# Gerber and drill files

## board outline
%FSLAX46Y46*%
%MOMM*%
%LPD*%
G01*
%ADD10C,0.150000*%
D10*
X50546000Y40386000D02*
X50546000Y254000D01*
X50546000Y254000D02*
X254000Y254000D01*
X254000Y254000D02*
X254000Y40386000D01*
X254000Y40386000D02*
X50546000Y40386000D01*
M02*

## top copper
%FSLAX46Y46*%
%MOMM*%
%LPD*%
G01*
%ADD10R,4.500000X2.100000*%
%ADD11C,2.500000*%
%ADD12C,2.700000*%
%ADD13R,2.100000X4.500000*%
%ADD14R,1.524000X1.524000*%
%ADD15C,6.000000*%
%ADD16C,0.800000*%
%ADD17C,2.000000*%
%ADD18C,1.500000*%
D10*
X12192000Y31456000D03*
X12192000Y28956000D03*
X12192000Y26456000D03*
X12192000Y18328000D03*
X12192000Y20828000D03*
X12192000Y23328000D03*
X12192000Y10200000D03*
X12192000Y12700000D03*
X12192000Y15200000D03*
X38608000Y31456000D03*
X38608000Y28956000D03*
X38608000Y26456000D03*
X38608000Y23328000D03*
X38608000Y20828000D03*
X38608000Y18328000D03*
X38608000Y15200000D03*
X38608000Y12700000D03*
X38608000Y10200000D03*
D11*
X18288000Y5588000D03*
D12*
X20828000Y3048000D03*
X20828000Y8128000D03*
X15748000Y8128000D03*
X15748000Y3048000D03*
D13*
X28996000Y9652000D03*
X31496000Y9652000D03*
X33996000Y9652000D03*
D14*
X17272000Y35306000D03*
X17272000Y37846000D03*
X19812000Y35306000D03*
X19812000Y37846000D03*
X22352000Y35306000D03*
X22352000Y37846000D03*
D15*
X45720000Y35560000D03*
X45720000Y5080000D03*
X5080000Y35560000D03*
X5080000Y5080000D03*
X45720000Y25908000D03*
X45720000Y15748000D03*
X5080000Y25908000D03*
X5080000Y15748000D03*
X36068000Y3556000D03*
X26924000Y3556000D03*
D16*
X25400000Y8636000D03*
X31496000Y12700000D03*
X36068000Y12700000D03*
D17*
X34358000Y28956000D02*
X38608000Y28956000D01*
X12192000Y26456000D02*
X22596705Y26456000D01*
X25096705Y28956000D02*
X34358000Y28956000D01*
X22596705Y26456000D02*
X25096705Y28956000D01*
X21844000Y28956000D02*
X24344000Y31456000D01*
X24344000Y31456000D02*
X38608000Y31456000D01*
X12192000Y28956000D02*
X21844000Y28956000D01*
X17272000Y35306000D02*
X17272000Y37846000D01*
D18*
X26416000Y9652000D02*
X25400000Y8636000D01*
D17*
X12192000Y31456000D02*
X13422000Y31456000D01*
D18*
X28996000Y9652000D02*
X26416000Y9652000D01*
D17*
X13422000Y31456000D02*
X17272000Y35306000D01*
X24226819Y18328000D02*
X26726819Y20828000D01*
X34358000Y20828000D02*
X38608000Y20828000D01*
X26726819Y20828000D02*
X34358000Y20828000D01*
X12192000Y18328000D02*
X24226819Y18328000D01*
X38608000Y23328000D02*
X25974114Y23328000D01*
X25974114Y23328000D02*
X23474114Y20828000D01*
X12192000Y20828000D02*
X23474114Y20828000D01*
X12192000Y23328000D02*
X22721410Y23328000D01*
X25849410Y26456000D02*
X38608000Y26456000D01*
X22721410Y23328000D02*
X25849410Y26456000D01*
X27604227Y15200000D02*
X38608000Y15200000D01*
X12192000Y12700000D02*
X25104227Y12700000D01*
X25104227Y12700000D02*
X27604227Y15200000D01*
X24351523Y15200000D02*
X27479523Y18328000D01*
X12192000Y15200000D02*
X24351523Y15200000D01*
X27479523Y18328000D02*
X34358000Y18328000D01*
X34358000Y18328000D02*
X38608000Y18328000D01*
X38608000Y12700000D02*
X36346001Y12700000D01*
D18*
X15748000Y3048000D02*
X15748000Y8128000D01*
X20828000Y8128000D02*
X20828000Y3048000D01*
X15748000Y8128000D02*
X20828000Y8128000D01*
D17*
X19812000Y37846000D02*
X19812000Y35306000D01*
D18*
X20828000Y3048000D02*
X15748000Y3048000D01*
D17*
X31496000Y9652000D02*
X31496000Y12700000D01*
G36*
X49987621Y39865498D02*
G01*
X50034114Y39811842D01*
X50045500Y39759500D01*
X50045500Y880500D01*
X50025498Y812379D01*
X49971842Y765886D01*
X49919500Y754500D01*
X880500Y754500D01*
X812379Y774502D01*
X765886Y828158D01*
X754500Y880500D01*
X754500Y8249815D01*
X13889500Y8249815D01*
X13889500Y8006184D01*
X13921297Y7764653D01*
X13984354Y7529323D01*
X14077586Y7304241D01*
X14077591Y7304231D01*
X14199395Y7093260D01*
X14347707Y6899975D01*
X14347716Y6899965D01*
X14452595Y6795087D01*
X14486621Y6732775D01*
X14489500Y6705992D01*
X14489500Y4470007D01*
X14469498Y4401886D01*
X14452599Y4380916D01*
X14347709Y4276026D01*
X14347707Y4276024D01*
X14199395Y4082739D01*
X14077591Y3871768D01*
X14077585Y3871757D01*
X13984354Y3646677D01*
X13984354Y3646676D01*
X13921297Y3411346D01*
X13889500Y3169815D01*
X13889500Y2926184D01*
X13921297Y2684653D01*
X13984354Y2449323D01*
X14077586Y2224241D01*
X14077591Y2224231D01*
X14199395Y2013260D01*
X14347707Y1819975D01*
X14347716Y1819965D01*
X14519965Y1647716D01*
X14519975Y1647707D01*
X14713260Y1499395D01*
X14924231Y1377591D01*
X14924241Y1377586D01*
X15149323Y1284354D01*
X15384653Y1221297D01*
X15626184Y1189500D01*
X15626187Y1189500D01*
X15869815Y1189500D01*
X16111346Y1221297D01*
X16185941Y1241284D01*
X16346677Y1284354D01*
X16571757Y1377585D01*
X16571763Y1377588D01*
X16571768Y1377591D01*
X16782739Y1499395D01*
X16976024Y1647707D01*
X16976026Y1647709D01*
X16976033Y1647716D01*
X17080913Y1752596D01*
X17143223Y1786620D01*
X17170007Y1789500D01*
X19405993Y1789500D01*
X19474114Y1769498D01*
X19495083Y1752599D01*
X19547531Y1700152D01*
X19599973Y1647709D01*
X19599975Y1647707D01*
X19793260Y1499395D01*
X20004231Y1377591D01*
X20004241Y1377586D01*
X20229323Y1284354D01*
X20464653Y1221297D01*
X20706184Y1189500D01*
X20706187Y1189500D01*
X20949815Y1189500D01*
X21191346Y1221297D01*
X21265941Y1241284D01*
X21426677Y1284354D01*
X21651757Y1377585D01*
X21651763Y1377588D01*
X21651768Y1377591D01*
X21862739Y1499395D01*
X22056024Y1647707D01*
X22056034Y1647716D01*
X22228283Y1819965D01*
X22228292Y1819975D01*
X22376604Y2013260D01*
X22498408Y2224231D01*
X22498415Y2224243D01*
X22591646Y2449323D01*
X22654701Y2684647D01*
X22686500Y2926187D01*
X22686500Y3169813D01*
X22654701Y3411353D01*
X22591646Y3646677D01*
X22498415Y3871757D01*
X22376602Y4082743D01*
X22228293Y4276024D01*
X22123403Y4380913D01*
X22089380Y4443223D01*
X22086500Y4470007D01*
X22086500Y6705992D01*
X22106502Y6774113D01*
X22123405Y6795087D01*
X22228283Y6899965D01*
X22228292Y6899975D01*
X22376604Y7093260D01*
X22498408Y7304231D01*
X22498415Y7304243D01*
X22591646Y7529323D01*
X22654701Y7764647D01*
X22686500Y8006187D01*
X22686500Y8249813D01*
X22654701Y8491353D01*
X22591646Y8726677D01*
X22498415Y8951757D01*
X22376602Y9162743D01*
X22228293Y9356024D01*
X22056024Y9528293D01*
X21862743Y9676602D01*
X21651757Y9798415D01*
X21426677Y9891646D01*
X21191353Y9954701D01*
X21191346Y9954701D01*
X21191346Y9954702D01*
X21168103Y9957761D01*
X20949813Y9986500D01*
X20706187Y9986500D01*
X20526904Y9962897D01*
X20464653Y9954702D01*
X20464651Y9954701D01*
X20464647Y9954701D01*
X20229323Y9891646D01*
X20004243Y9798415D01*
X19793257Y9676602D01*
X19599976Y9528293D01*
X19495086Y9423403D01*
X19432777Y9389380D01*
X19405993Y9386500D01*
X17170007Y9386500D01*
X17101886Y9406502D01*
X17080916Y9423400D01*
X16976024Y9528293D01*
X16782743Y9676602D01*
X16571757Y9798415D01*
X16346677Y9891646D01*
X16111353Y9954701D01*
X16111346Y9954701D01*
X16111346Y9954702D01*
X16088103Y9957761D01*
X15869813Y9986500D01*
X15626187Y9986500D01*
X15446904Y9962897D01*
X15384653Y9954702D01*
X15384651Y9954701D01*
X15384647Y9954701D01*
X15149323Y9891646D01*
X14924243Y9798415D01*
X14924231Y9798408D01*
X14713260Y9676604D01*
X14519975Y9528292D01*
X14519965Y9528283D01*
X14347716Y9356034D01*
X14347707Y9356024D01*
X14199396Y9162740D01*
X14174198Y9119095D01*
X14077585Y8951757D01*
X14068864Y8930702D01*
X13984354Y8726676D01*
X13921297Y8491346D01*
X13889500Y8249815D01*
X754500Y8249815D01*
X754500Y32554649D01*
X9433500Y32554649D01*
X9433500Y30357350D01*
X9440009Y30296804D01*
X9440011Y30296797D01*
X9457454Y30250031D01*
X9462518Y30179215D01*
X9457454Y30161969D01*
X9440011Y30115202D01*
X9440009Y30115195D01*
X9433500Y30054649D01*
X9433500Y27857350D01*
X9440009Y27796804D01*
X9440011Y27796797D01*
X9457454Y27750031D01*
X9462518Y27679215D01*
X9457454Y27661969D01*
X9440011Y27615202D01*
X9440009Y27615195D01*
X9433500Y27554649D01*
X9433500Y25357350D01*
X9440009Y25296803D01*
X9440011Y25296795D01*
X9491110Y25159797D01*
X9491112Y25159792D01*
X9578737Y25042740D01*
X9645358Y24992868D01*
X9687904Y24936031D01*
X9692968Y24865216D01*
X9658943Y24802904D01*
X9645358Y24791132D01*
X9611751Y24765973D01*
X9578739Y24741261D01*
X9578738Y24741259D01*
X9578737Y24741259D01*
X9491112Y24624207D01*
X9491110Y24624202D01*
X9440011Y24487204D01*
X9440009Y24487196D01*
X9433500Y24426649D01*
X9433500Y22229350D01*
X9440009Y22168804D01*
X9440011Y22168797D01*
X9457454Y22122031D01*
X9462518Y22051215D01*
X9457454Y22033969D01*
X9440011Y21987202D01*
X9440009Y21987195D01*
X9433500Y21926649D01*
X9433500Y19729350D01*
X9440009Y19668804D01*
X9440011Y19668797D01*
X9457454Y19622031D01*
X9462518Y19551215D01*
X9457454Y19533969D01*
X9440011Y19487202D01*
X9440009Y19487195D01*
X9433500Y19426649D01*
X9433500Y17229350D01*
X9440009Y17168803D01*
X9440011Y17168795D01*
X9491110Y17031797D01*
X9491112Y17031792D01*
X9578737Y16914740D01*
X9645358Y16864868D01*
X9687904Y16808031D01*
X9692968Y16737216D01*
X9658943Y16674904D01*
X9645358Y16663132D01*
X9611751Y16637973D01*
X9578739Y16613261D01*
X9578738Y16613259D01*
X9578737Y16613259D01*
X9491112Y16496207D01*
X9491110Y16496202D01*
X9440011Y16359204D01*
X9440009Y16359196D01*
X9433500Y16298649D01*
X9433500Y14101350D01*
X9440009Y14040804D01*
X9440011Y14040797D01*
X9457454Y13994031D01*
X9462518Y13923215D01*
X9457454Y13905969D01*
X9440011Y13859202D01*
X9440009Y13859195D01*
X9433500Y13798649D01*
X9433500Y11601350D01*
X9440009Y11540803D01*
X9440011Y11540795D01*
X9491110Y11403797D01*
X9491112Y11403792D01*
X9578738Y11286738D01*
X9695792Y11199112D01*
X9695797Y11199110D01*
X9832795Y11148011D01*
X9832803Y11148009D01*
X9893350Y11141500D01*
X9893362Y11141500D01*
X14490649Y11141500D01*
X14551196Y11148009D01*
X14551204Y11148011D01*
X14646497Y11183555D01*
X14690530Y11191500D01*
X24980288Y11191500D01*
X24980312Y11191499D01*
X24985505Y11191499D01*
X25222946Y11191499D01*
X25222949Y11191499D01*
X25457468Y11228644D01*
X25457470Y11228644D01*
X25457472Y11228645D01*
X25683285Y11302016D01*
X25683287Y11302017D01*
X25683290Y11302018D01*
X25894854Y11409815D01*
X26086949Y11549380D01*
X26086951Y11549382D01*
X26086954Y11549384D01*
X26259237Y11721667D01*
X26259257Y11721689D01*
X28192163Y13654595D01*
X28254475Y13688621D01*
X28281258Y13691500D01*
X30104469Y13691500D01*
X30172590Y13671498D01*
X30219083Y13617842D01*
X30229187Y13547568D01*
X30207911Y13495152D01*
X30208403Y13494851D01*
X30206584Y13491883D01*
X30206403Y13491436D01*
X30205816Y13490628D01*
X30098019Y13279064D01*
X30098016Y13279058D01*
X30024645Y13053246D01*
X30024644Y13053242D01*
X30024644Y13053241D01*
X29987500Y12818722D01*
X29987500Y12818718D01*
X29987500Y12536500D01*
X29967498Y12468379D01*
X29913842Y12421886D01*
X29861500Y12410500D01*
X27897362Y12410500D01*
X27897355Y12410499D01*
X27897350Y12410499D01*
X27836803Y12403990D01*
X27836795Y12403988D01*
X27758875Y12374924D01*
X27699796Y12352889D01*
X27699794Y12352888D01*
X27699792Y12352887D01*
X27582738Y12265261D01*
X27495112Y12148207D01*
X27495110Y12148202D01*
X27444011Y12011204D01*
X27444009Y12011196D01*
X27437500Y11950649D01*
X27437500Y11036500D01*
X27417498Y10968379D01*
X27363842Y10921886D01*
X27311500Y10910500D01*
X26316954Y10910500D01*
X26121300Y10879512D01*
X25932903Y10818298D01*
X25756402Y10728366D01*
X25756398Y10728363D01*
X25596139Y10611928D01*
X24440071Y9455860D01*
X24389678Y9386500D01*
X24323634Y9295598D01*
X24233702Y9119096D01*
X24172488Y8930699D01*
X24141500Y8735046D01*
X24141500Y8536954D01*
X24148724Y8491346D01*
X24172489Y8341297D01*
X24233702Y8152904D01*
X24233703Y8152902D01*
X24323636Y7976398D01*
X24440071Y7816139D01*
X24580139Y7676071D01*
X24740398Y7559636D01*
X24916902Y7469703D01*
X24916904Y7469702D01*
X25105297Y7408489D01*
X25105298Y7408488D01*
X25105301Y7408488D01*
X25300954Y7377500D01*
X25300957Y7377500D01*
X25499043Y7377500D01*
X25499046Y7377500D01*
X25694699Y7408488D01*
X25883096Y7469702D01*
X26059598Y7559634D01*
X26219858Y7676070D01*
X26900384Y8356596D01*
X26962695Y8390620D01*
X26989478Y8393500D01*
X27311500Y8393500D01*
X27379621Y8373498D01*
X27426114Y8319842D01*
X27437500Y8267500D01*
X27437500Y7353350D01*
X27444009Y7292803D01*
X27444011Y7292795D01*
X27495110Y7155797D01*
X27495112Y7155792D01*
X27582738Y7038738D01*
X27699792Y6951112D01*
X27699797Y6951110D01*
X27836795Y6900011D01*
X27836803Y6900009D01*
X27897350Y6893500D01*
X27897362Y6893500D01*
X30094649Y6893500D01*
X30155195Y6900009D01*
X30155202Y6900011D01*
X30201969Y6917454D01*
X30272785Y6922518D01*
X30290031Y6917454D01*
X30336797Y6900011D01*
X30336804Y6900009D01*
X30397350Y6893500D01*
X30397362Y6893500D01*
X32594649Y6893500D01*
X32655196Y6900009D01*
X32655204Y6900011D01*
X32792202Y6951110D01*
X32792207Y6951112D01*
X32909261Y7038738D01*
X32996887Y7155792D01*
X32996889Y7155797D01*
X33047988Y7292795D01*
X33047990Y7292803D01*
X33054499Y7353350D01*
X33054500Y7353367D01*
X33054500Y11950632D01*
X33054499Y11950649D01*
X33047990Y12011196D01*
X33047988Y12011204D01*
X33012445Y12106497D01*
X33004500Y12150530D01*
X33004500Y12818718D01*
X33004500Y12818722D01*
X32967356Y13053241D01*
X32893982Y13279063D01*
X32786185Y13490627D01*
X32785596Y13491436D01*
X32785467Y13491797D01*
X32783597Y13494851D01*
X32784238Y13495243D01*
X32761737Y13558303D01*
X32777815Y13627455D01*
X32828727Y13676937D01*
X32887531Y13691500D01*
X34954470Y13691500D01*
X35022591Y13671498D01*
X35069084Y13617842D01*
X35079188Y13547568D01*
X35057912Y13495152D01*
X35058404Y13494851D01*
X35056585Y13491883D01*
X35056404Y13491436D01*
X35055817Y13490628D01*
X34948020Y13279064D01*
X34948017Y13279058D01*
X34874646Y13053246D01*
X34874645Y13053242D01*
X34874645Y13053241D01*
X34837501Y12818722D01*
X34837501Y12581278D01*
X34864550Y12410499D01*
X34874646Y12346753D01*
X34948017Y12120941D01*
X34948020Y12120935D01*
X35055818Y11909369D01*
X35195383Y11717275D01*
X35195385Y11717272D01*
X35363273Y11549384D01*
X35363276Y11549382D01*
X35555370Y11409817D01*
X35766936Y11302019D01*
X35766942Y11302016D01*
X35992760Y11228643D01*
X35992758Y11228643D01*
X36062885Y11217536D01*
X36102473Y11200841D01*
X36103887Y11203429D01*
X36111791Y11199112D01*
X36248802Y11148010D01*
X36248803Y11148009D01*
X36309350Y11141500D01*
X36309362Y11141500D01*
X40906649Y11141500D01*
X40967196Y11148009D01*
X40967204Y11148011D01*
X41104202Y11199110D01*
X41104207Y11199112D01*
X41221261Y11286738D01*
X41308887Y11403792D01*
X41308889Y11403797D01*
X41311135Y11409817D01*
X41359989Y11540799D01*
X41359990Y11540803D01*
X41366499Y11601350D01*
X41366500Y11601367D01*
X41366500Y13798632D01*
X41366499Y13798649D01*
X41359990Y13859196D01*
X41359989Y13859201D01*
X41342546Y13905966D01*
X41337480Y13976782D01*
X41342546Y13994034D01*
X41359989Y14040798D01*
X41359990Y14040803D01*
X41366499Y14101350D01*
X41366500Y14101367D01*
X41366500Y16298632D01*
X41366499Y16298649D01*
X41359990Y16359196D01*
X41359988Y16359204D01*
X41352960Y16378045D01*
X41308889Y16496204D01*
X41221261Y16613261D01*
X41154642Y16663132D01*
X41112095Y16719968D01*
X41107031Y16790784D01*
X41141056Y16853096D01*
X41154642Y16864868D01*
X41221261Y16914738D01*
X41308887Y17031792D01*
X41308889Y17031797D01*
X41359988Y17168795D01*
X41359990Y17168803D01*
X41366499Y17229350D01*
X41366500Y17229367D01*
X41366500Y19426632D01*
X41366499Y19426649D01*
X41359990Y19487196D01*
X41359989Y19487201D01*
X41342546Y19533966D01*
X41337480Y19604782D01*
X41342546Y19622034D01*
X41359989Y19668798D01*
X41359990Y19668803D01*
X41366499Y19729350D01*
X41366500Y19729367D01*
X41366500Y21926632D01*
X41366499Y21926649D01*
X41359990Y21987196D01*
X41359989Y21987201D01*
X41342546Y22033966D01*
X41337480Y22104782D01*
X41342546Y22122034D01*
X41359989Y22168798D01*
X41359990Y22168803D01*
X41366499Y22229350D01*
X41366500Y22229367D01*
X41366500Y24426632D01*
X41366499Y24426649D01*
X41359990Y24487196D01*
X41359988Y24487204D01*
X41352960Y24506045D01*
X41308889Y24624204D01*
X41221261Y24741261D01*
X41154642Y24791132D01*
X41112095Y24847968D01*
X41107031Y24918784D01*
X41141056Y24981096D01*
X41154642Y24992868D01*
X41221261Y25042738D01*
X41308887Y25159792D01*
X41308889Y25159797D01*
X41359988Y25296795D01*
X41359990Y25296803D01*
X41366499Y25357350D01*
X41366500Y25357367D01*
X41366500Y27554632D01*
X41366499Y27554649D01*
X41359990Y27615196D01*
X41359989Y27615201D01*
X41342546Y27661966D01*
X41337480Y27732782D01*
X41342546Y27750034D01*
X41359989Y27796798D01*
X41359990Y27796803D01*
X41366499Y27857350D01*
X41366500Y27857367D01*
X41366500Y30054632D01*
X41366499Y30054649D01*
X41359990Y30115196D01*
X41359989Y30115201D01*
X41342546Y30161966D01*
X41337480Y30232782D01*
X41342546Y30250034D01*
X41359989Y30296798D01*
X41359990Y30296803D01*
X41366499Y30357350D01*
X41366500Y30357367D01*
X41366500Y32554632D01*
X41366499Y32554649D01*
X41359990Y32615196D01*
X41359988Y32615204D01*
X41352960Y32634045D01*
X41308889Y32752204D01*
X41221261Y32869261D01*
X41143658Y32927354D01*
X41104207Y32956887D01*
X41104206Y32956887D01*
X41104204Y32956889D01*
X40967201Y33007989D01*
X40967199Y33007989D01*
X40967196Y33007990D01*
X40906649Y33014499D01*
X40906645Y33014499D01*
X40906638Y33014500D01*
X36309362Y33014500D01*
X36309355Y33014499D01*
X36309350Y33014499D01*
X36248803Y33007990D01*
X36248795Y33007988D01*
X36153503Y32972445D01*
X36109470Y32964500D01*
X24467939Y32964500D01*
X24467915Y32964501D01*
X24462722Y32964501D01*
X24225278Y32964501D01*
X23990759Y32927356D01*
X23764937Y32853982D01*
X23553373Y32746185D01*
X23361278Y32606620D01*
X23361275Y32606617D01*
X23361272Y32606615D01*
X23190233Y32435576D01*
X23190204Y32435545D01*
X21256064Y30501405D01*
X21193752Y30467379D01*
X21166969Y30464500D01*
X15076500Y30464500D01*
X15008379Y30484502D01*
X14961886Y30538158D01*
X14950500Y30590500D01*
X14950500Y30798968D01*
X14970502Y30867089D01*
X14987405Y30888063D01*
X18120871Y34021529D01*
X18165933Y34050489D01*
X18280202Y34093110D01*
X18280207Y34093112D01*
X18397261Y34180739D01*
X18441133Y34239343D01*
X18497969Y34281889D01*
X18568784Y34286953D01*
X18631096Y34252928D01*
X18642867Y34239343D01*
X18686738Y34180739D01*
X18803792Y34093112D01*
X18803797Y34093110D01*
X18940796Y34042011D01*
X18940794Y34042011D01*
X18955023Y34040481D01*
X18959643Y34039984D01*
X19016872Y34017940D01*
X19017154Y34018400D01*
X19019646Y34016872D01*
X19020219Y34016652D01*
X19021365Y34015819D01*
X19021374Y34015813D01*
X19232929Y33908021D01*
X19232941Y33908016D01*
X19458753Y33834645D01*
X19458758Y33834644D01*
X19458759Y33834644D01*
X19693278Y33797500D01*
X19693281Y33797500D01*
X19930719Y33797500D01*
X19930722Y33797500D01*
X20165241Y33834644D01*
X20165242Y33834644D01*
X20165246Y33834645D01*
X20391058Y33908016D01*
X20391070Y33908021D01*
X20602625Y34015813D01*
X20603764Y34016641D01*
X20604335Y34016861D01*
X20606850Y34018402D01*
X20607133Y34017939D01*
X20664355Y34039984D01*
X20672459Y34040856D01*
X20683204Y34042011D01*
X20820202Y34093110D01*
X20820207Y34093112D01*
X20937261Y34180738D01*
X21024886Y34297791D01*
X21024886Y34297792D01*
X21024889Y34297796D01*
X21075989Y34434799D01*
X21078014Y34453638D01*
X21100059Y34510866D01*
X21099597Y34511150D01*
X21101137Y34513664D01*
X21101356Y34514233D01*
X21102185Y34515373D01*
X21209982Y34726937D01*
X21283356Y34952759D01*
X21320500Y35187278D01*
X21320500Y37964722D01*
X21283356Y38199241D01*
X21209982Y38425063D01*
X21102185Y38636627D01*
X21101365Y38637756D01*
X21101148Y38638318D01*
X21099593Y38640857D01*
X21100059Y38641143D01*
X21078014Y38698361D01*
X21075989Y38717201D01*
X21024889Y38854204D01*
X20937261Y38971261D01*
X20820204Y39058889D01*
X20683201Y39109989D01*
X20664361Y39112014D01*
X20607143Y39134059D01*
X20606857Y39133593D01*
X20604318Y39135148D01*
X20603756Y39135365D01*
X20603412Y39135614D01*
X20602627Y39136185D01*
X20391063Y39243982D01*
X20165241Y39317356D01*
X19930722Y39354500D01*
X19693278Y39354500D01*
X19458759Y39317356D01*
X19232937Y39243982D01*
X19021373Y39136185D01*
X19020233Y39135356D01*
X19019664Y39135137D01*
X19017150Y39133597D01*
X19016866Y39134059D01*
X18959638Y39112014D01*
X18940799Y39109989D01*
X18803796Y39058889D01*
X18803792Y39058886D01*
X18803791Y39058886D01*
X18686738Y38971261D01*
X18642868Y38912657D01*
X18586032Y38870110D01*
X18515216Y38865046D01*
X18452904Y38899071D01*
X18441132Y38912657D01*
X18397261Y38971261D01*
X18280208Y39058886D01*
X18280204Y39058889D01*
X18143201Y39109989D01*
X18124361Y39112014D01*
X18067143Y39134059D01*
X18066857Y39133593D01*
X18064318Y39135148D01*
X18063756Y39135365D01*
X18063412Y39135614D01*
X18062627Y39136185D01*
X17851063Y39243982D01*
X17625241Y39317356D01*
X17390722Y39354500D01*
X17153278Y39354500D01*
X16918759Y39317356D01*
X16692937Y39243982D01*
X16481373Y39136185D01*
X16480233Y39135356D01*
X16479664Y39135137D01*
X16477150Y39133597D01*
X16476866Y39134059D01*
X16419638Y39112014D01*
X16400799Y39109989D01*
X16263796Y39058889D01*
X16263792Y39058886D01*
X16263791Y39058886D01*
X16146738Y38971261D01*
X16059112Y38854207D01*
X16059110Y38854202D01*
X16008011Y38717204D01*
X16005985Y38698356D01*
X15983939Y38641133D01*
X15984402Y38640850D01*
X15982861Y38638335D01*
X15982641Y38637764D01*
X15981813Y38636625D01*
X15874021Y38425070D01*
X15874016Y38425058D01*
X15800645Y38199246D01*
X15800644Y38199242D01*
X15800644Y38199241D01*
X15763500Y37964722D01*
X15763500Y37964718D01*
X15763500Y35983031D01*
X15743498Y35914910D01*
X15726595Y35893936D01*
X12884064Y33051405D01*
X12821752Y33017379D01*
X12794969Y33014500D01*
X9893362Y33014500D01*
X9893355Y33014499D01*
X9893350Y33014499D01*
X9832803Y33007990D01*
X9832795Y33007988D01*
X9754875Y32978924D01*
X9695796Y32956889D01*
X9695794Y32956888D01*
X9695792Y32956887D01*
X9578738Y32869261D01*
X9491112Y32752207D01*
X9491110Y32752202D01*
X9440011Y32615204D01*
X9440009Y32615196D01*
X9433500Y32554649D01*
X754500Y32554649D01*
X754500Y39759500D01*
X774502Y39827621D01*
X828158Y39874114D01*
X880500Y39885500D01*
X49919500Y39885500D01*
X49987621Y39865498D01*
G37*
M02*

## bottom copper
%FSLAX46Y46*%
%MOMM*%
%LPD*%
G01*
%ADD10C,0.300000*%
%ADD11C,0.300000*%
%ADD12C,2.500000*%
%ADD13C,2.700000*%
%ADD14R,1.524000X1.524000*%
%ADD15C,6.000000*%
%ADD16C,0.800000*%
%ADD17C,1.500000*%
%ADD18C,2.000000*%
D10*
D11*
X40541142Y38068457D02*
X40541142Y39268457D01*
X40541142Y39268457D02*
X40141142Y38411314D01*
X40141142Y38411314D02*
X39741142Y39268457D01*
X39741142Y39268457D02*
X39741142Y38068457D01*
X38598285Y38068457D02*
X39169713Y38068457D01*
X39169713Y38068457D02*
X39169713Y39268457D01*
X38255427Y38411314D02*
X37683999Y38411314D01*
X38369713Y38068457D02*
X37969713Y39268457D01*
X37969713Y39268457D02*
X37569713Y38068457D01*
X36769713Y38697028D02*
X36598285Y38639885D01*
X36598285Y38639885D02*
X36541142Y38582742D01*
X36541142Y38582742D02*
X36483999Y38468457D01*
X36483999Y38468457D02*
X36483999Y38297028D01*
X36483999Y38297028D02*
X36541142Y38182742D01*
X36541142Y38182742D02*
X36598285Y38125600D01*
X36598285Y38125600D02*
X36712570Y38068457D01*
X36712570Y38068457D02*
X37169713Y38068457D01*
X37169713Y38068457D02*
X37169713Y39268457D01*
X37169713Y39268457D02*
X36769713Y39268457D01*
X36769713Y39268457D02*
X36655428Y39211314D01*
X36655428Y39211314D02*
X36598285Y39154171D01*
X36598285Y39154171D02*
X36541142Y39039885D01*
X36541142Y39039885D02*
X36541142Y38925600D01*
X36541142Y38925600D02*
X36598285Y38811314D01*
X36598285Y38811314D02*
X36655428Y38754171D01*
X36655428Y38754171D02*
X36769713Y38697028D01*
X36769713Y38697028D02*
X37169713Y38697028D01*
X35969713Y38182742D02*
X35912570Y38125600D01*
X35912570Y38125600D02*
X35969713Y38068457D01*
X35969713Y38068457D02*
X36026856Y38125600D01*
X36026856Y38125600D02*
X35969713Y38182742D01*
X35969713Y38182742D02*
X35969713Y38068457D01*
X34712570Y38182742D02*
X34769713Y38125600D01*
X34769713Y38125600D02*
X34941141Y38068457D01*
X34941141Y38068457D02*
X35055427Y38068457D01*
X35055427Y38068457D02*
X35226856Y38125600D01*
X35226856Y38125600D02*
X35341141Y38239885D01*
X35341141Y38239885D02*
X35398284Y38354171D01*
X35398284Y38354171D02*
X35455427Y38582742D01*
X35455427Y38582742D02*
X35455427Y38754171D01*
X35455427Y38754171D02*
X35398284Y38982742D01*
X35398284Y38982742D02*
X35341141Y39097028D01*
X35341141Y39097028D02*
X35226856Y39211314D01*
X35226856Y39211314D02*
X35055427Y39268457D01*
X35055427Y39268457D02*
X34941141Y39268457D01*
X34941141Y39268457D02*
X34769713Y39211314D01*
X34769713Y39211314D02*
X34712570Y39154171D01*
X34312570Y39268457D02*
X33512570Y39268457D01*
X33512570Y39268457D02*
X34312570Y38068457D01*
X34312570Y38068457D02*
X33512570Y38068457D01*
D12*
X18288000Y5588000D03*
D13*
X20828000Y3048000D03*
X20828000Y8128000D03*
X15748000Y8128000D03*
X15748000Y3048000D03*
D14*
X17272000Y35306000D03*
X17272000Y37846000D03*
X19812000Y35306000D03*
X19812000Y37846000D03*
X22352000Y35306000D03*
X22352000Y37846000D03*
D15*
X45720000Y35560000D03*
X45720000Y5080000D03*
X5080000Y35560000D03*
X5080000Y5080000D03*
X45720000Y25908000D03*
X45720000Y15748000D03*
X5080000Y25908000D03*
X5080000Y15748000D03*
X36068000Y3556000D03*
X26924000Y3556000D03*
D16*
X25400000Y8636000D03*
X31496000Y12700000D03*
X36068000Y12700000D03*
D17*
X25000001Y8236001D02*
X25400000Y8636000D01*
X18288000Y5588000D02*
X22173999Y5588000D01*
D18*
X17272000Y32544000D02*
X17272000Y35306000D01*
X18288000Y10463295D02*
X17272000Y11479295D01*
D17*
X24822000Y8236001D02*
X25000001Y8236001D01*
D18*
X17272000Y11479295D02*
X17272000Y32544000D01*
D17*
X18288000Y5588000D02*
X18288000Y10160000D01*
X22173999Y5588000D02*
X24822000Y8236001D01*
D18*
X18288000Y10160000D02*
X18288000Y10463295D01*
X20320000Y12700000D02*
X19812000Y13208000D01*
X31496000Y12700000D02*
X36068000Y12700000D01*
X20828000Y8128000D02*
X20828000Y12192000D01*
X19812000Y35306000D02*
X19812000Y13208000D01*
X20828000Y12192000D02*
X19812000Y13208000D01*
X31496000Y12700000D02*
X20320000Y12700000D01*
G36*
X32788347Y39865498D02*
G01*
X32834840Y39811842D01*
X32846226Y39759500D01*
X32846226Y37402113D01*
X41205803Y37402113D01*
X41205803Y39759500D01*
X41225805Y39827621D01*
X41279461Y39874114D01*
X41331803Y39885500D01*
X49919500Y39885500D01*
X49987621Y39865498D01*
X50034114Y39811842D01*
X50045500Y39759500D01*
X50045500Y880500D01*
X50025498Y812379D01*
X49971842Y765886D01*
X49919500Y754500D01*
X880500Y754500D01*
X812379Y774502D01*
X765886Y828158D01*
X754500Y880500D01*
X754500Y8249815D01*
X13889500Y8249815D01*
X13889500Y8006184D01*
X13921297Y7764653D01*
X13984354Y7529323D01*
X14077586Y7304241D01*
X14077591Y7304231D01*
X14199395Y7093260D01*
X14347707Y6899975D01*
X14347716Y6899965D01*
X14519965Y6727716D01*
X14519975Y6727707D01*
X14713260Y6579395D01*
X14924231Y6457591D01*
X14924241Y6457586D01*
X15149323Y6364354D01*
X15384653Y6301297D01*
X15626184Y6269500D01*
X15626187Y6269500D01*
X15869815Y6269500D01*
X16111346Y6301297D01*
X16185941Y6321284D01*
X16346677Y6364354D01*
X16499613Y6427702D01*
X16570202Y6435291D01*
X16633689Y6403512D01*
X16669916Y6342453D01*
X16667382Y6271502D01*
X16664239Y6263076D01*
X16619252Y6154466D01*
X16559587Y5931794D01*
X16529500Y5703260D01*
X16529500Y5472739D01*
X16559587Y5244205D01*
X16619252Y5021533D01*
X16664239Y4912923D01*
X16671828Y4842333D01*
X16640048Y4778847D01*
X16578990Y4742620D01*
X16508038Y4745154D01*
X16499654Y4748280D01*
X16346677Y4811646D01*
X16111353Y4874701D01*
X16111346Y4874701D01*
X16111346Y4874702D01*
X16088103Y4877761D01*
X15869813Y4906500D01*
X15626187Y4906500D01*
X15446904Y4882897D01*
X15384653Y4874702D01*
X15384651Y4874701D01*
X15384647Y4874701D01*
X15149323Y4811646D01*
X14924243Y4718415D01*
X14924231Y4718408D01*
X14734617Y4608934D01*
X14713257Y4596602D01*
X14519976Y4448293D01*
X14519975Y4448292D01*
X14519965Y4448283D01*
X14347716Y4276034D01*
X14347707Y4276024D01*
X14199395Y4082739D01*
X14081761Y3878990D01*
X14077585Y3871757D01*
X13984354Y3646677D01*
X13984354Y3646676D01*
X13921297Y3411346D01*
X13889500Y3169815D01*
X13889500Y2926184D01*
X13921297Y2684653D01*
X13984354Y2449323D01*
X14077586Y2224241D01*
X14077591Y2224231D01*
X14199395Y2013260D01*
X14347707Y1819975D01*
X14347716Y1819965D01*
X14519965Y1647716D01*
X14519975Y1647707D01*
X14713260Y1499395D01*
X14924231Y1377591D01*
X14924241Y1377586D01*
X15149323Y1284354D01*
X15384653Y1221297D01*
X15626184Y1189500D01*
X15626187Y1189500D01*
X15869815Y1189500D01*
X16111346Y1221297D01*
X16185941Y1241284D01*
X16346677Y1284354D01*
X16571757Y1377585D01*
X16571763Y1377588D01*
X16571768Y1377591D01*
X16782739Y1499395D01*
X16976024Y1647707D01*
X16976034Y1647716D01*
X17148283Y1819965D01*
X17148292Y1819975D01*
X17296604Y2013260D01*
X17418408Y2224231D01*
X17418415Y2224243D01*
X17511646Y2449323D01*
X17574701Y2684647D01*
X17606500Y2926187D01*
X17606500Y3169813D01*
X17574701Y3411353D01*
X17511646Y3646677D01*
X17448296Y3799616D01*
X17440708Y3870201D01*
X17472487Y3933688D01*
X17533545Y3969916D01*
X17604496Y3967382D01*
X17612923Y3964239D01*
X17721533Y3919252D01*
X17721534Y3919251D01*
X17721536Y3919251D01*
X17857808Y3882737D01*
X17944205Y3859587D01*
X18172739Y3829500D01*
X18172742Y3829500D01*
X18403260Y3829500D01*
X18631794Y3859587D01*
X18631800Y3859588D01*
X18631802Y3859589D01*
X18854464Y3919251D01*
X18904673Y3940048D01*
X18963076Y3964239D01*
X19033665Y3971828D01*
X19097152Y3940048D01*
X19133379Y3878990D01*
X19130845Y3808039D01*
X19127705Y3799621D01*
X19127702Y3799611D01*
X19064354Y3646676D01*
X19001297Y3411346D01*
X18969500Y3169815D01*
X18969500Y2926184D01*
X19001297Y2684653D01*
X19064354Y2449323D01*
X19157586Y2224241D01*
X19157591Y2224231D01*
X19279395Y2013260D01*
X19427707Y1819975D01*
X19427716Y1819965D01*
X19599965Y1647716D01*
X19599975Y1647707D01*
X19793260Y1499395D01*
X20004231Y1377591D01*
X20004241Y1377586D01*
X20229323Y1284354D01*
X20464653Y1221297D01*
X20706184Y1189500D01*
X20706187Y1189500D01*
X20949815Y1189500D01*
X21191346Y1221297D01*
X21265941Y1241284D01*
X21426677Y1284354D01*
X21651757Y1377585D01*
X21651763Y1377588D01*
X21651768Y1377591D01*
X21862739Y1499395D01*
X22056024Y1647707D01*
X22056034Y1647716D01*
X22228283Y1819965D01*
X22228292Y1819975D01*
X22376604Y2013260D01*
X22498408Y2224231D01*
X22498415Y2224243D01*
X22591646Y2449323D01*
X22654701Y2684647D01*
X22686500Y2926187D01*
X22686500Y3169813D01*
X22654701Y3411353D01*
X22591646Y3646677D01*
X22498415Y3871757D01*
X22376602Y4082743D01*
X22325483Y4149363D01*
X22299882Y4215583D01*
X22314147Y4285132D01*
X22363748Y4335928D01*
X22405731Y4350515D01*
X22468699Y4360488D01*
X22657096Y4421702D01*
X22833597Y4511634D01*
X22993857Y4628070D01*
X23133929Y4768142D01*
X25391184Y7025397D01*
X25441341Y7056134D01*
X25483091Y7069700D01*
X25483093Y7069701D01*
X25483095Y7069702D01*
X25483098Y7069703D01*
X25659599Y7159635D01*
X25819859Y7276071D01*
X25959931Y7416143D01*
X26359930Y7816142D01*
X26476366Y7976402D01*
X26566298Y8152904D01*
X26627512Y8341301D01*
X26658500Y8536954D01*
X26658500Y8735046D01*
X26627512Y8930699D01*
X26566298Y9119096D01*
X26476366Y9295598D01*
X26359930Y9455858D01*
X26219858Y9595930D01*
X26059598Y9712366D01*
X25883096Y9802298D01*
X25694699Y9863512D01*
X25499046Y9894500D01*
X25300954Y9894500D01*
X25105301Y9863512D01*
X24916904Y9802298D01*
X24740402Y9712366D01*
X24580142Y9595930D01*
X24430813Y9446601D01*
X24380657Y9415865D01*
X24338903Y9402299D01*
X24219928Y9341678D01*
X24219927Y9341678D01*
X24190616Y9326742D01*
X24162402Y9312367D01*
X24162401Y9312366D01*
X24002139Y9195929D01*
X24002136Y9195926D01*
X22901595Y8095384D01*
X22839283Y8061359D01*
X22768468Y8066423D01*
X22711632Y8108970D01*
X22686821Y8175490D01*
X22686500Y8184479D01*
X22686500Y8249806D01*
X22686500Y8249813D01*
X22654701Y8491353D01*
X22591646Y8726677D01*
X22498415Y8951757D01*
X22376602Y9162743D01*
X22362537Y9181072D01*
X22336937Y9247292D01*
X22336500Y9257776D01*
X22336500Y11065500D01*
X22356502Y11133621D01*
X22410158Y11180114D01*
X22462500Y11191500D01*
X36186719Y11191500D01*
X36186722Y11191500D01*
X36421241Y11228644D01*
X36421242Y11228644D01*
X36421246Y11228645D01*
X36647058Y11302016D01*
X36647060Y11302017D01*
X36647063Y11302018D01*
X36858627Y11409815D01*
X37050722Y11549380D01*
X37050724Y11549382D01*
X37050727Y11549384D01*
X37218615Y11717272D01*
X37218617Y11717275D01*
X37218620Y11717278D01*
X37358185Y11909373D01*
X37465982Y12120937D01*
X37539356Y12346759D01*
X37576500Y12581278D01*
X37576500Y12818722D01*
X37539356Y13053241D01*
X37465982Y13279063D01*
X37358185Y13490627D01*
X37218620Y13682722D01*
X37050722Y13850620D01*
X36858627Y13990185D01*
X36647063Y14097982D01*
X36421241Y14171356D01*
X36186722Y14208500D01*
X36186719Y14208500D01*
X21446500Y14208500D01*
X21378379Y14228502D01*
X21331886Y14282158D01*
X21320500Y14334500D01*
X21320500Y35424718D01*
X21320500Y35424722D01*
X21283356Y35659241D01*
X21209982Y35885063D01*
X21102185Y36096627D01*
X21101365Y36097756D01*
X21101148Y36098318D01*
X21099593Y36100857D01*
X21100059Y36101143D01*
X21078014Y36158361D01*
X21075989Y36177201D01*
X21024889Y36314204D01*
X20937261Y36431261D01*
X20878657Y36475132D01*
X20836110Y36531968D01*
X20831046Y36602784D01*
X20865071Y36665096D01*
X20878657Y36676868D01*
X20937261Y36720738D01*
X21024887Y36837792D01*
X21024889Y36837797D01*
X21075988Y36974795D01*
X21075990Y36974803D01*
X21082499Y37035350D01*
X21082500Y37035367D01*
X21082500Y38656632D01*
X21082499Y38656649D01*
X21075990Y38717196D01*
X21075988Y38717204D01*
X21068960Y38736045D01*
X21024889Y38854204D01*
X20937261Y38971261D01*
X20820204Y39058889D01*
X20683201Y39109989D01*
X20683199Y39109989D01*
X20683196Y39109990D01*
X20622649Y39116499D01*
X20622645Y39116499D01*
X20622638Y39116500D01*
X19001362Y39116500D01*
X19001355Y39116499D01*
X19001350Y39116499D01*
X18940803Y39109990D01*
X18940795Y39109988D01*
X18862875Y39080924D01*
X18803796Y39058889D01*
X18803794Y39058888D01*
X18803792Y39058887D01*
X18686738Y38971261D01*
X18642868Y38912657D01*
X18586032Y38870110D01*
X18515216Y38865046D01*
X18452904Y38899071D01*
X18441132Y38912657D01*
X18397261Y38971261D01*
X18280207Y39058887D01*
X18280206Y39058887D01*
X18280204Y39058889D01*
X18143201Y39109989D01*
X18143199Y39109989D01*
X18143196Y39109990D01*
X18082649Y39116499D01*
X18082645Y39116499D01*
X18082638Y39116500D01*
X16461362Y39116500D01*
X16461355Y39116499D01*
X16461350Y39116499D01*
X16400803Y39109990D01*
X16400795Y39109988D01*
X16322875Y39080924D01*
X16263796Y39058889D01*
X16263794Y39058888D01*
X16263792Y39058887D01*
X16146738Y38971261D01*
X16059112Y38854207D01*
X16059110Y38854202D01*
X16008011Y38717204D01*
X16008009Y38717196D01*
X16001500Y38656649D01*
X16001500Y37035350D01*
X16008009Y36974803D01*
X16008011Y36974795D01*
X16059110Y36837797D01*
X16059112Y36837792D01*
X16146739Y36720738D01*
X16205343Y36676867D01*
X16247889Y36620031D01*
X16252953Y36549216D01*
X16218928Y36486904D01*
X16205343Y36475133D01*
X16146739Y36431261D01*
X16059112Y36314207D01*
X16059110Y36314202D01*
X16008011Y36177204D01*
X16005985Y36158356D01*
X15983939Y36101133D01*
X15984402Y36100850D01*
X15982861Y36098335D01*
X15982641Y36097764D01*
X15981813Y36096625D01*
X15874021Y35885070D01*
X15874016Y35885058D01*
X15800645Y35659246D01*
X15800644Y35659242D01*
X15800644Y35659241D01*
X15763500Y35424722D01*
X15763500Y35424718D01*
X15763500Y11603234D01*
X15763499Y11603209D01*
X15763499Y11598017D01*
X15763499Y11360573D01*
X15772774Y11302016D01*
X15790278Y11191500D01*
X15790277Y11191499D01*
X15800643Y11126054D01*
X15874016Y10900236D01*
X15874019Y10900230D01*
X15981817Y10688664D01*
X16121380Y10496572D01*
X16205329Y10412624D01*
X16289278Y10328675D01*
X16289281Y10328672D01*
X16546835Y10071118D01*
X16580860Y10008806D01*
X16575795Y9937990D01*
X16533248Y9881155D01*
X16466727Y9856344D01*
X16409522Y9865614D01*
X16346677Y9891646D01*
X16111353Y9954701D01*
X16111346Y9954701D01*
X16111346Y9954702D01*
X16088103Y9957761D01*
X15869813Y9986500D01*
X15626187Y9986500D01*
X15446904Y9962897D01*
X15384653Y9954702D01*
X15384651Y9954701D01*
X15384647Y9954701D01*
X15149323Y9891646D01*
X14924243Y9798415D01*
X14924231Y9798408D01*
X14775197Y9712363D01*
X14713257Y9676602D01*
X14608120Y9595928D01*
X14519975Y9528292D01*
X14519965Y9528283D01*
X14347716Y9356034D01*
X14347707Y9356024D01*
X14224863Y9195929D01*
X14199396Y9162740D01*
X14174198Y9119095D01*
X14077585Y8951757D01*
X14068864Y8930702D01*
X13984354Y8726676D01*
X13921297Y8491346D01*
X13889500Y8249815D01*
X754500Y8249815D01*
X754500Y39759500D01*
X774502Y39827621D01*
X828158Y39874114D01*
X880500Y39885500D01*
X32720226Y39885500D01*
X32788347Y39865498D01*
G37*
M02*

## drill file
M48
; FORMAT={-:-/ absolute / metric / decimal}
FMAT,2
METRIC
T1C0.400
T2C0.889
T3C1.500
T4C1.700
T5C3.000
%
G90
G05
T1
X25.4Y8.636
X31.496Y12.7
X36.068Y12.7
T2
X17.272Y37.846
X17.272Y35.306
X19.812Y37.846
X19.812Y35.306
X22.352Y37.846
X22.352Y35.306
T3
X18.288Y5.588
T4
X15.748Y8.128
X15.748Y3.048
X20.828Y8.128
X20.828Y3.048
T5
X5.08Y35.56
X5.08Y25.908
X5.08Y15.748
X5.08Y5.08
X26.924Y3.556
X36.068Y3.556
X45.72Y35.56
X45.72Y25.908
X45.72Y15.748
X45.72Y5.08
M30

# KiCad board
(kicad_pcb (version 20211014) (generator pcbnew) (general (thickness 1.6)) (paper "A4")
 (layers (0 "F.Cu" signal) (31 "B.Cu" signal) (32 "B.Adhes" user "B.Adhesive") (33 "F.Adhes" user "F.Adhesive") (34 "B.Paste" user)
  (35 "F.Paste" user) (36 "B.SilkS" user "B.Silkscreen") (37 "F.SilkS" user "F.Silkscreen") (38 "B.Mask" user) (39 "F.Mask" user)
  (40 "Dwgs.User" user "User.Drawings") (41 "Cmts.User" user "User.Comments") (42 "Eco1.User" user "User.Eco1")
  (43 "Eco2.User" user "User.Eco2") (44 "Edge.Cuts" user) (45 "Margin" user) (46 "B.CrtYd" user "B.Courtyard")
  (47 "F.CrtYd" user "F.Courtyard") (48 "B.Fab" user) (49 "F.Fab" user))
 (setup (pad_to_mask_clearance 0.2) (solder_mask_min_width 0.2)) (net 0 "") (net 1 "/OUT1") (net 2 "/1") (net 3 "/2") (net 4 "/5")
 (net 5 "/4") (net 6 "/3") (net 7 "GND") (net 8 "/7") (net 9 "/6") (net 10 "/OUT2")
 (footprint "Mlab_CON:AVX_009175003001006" (layer "F.Cu") (at 12.192 -28.956 -90)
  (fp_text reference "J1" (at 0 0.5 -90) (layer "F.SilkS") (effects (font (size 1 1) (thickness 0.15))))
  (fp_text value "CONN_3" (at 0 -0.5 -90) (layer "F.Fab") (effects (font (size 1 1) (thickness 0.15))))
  (pad "1" smd rect locked (at -2.5 0 270) (size 2.1 4.5) (layers "F.Cu" "F.Paste" "F.Mask") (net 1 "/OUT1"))
  (pad "2" smd rect locked (at 0 0 270) (size 2.1 4.5) (layers "F.Cu" "F.Paste" "F.Mask") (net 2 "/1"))
  (pad "3" smd rect locked (at 2.5 0 270) (size 2.1 4.5) (layers "F.Cu" "F.Paste" "F.Mask") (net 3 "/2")))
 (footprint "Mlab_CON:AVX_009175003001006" (layer "F.Cu") (at 12.192 -20.828 90)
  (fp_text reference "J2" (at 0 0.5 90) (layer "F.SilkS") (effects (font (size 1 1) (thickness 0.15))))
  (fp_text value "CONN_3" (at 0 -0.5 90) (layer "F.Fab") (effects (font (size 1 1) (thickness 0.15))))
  (pad "1" smd rect locked (at -2.5 0 90) (size 2.1 4.5) (layers "F.Cu" "F.Paste" "F.Mask") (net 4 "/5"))
  (pad "2" smd rect locked (at 0 0 90) (size 2.1 4.5) (layers "F.Cu" "F.Paste" "F.Mask") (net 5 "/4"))
  (pad "3" smd rect locked (at 2.5 0 90) (size 2.1 4.5) (layers "F.Cu" "F.Paste" "F.Mask") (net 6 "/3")))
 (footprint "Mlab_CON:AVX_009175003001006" (layer "F.Cu") (at 12.192 -12.7 90)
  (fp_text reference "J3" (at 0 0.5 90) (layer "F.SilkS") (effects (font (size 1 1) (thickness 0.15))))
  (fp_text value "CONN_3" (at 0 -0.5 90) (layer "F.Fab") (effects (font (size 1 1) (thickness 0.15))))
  (pad "1" smd rect locked (at -2.5 0 90) (size 2.1 4.5) (layers "F.Cu" "F.Paste" "F.Mask") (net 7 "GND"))
  (pad "2" smd rect locked (at 0 0 90) (size 2.1 4.5) (layers "F.Cu" "F.Paste" "F.Mask") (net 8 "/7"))
  (pad "3" smd rect locked (at 2.5 0 90) (size 2.1 4.5) (layers "F.Cu" "F.Paste" "F.Mask") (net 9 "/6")))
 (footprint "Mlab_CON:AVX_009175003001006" (layer "F.Cu") (at 38.608 -28.956 -90)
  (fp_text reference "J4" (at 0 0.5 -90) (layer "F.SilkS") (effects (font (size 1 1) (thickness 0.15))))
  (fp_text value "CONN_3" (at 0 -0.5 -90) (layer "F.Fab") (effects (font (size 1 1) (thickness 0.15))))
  (pad "1" smd rect locked (at -2.5 0 270) (size 2.1 4.5) (layers "F.Cu" "F.Paste" "F.Mask") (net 2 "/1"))
  (pad "2" smd rect locked (at 0 0 270) (size 2.1 4.5) (layers "F.Cu" "F.Paste" "F.Mask") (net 3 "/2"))
  (pad "3" smd rect locked (at 2.5 0 270) (size 2.1 4.5) (layers "F.Cu" "F.Paste" "F.Mask") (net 6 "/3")))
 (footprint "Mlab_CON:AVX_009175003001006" (layer "F.Cu") (at 38.608 -20.828 -90)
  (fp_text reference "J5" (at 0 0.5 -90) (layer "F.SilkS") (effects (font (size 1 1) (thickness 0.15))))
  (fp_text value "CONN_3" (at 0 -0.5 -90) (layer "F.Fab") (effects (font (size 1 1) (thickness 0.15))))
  (pad "1" smd rect locked (at -2.5 0 270) (size 2.1 4.5) (layers "F.Cu" "F.Paste" "F.Mask") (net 5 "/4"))
  (pad "2" smd rect locked (at 0 0 270) (size 2.1 4.5) (layers "F.Cu" "F.Paste" "F.Mask") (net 4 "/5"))
  (pad "3" smd rect locked (at 2.5 0 270) (size 2.1 4.5) (layers "F.Cu" "F.Paste" "F.Mask") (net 9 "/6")))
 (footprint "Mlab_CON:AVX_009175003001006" (layer "F.Cu") (at 38.608 -12.7 -90)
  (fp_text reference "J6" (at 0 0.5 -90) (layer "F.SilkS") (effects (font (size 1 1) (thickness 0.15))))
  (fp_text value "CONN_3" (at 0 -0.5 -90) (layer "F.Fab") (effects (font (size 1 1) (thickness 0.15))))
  (pad "1" smd rect locked (at -2.5 0 270) (size 2.1 4.5) (layers "F.Cu" "F.Paste" "F.Mask") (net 8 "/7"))
  (pad "2" smd rect locked (at 0 0 270) (size 2.1 4.5) (layers "F.Cu" "F.Paste" "F.Mask") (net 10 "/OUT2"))
  (pad "3" smd rect locked (at 2.5 0 270) (size 2.1 4.5) (layers "F.Cu" "F.Paste" "F.Mask") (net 7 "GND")))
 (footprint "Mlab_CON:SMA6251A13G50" (layer "F.Cu") (at 18.288 -5.588)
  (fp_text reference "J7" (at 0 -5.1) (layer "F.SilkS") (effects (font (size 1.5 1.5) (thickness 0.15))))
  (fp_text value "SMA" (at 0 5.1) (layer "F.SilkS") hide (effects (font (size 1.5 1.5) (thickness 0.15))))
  (pad "1" thru_hole circle locked (at 0 0 180) (size 2.5 2.5) (drill 1.5) (layers *.Cu *.Mask) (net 1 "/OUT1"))
  (pad "2" thru_hole circle locked (at 2.54 2.54 180) (size 2.7 2.7) (drill 1.7) (layers *.Cu *.Mask) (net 10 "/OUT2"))
  (pad "2" thru_hole circle locked (at 2.54 -2.54 180) (size 2.7 2.7) (drill 1.7) (layers *.Cu *.Mask) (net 10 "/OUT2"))
  (pad "2" thru_hole circle locked (at -2.54 -2.54 180) (size 2.7 2.7) (drill 1.7) (layers *.Cu *.Mask) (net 10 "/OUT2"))
  (pad "2" thru_hole circle locked (at -2.54 2.54 180) (size 2.7 2.7) (drill 1.7) (layers *.Cu *.Mask) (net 10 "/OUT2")))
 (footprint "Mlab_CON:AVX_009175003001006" (layer "F.Cu") (at 31.496 -9.652)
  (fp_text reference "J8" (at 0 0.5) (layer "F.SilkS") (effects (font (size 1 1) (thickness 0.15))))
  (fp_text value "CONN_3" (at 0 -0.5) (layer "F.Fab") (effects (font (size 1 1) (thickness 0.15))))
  (pad "1" smd rect locked (at -2.5 0) (size 2.1 4.5) (layers "F.Cu" "F.Paste" "F.Mask") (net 1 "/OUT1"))
  (pad "2" smd rect locked (at 0 0) (size 2.1 4.5) (layers "F.Cu" "F.Paste" "F.Mask") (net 10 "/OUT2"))
  (pad "3" smd rect locked (at 2.5 0) (size 2.1 4.5) (layers "F.Cu" "F.Paste" "F.Mask") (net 7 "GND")))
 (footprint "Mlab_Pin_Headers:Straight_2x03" (layer "F.Cu") (at 19.812 -36.576 90)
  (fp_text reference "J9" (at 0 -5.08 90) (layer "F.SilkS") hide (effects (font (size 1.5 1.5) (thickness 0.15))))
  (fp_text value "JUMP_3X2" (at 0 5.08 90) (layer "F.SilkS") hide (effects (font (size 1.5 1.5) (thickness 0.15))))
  (pad "1" thru_hole rect locked (at -1.27 -2.54 90) (size 1.524 1.524) (drill 0.889) (layers *.Cu *.Mask "F.SilkS") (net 1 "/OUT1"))
  (pad "2" thru_hole rect locked (at 1.27 -2.54 90) (size 1.524 1.524) (drill 0.889) (layers *.Cu *.Mask "F.SilkS") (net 1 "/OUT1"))
  (pad "3" thru_hole rect locked (at -1.27 0 90) (size 1.524 1.524) (drill 0.889) (layers *.Cu *.Mask "F.SilkS") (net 10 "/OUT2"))
  (pad "4" thru_hole rect locked (at 1.27 0 90) (size 1.524 1.524) (drill 0.889) (layers *.Cu *.Mask "F.SilkS") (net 10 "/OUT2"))
  (pad "5" thru_hole rect locked (at -1.27 2.54 90) (size 1.524 1.524) (drill 0.889) (layers *.Cu *.Mask "F.SilkS") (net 7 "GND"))
  (pad "6" thru_hole rect locked (at 1.27 2.54 90) (size 1.524 1.524) (drill 0.889) (layers *.Cu *.Mask "F.SilkS") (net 7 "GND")))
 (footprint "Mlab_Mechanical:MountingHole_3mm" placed (layer "F.Cu") (at 45.72 -35.56)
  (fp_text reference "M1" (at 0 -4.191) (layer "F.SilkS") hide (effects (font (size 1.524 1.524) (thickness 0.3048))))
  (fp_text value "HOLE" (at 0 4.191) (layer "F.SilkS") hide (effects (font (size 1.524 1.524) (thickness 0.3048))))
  (pad "1" thru_hole circle locked (at 0 0) (size 6 6) (drill 3) (layers *.Cu *.Adhes *.Mask) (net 7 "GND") (clearance 1) (zone_connect 2)))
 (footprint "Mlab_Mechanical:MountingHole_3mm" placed (layer "F.Cu") (at 45.72 -5.08)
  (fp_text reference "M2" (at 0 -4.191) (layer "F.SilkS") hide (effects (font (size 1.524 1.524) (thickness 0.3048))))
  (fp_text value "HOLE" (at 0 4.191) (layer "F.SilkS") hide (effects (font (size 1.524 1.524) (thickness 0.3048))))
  (pad "1" thru_hole circle locked (at 0 0) (size 6 6) (drill 3) (layers *.Cu *.Adhes *.Mask) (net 7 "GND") (clearance 1) (zone_connect 2)))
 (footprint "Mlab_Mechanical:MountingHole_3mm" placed (layer "F.Cu") (at 5.08 -35.56)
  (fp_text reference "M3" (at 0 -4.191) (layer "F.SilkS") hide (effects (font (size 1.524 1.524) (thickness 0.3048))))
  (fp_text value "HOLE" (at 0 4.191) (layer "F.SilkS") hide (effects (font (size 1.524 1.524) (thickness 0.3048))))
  (pad "1" thru_hole circle locked (at 0 0) (size 6 6) (drill 3) (layers *.Cu *.Adhes *.Mask) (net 7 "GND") (clearance 1) (zone_connect 2)))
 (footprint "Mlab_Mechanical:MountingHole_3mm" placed (layer "F.Cu") (at 5.08 -5.08)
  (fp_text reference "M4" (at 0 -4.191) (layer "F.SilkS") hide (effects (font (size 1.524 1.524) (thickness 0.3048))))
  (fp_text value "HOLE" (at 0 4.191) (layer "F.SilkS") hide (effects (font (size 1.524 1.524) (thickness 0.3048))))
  (pad "1" thru_hole circle locked (at 0 0) (size 6 6) (drill 3) (layers *.Cu *.Adhes *.Mask) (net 7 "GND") (clearance 1) (zone_connect 2)))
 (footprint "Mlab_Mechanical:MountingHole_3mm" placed (layer "F.Cu") (at 45.72 -25.908)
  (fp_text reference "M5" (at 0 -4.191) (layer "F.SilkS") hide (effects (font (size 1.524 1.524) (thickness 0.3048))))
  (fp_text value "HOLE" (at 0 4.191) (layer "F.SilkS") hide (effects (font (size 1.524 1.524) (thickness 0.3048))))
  (pad "1" thru_hole circle locked (at 0 0) (size 6 6) (drill 3) (layers *.Cu *.Adhes *.Mask) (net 7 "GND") (clearance 1) (zone_connect 2)))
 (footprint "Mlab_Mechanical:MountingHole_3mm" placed (layer "F.Cu") (at 45.72 -15.748)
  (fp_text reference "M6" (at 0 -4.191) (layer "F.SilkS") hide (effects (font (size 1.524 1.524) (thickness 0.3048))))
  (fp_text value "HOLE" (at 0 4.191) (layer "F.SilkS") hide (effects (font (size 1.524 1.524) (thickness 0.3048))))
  (pad "1" thru_hole circle locked (at 0 0) (size 6 6) (drill 3) (layers *.Cu *.Adhes *.Mask) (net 7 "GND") (clearance 1) (zone_connect 2)))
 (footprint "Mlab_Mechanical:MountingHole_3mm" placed (layer "F.Cu") (at 5.08 -25.908)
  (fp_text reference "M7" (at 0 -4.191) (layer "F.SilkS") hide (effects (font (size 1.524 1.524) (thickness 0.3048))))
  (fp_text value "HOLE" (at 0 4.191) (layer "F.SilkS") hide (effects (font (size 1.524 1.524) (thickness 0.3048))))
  (pad "1" thru_hole circle locked (at 0 0) (size 6 6) (drill 3) (layers *.Cu *.Adhes *.Mask) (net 7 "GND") (clearance 1) (zone_connect 2)))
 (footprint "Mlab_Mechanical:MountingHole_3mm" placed (layer "F.Cu") (at 5.08 -15.748)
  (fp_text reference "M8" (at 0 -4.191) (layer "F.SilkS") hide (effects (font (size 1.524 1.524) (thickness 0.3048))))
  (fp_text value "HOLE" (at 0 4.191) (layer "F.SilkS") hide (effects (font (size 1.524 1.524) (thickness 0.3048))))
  (pad "1" thru_hole circle locked (at 0 0) (size 6 6) (drill 3) (layers *.Cu *.Adhes *.Mask) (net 7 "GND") (clearance 1) (zone_connect 2)))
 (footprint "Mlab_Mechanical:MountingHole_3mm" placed (layer "F.Cu") (at 36.068 -3.556)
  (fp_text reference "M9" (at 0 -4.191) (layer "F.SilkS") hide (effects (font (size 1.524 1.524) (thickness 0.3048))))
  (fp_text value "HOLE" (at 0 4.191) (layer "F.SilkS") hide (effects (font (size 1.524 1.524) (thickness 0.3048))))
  (pad "1" thru_hole circle locked (at 0 0) (size 6 6) (drill 3) (layers *.Cu *.Adhes *.Mask) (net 7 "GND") (clearance 1) (zone_connect 2)))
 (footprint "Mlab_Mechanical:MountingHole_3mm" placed (layer "F.Cu") (at 26.924 -3.556)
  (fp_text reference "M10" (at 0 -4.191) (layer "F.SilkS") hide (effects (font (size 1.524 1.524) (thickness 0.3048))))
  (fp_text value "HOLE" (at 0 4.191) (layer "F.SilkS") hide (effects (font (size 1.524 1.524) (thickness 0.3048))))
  (pad "1" thru_hole circle locked (at 0 0) (size 6 6) (drill 3) (layers *.Cu *.Adhes *.Mask) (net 7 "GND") (clearance 1) (zone_connect 2)))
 (gr_line (start 50.546 -40.386) (end 50.546 -0.254) (layer "Edge.Cuts") (width 0.15))
 (gr_line (start 50.546 -0.254) (end 0.254 -0.254) (layer "Edge.Cuts") (width 0.15))
 (gr_line (start 0.254 -0.254) (end 0.254 -40.386) (layer "Edge.Cuts") (width 0.15))
 (gr_line (start 0.254 -40.386) (end 50.546 -40.386) (layer "Edge.Cuts") (width 0.15))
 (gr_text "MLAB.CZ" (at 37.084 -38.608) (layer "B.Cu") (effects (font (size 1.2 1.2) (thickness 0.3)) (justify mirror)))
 (segment (start 34.358 -28.956) (end 38.608 -28.956) (width 2) (layer "F.Cu") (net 3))
 (segment (start 12.192 -26.456) (end 22.596705 -26.456) (width 2) (layer "F.Cu") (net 3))
 (segment (start 25.096705 -28.956) (end 34.358 -28.956) (width 2) (layer "F.Cu") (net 3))
 (segment (start 22.596705 -26.456) (end 25.096705 -28.956) (width 2) (layer "F.Cu") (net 3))
 (segment (start 21.844 -28.956) (end 24.344 -31.456) (width 2) (layer "F.Cu") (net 2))
 (segment (start 24.344 -31.456) (end 38.608 -31.456) (width 2) (layer "F.Cu") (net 2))
 (segment (start 12.192 -28.956) (end 21.844 -28.956) (width 2) (layer "F.Cu") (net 2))
 (segment (start 17.272 -35.306) (end 17.272 -37.846) (width 2) (layer "F.Cu") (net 1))
 (segment (start 26.416 -9.652) (end 25.4 -8.636) (width 1.5) (layer "F.Cu") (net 1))
 (segment (start 12.192 -31.456) (end 13.422 -31.456) (width 2) (layer "F.Cu") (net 1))
 (segment (start 28.996 -9.652) (end 26.416 -9.652) (width 1.5) (layer "F.Cu") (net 1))
 (segment (start 13.422 -31.456) (end 17.272 -35.306) (width 2) (layer "F.Cu") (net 1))
 (via (at 25.4 -8.636) (size 0.8) (drill 0.4) (layers "F.Cu" "B.Cu") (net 1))
 (segment (start 25.000001 -8.236001) (end 25.4 -8.636) (width 1.5) (layer "B.Cu") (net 1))
 (segment (start 18.288 -5.588) (end 22.173999 -5.588) (width 1.5) (layer "B.Cu") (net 1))
 (segment (start 17.272 -32.544) (end 17.272 -35.306) (width 2) (layer "B.Cu") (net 1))
 (segment (start 18.288 -10.463295) (end 17.272 -11.479295) (width 2) (layer "B.Cu") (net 1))
 (segment (start 24.822 -8.236001) (end 25.000001 -8.236001) (width 1.5) (layer "B.Cu") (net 1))
 (segment (start 17.272 -11.479295) (end 17.272 -32.544) (width 2) (layer "B.Cu") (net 1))
 (segment (start 18.288 -5.588) (end 18.288 -10.16) (width 1.5) (layer "B.Cu") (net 1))
 (segment (start 22.173999 -5.588) (end 24.822 -8.236001) (width 1.5) (layer "B.Cu") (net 1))
 (segment (start 18.288 -10.16) (end 18.288 -10.463295) (width 2) (layer "B.Cu") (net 1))
 (segment (start 24.226819 -18.328) (end 26.726819 -20.828) (width 2) (layer "F.Cu") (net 4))
 (segment (start 34.358 -20.828) (end 38.608 -20.828) (width 2) (layer "F.Cu") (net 4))
 (segment (start 26.726819 -20.828) (end 34.358 -20.828) (width 2) (layer "F.Cu") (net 4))
 (segment (start 12.192 -18.328) (end 24.226819 -18.328) (width 2) (layer "F.Cu") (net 4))
 (segment (start 38.608 -23.328) (end 25.974114 -23.328) (width 2) (layer "F.Cu") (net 5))
 (segment (start 25.974114 -23.328) (end 23.474114 -20.828) (width 2) (layer "F.Cu") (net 5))
 (segment (start 12.192 -20.828) (end 23.474114 -20.828) (width 2) (layer "F.Cu") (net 5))
 (segment (start 12.192 -23.328) (end 22.72141 -23.328) (width 2) (layer "F.Cu") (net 6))
 (segment (start 25.84941 -26.456) (end 38.608 -26.456) (width 2) (layer "F.Cu") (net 6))
 (segment (start 22.72141 -23.328) (end 25.84941 -26.456) (width 2) (layer "F.Cu") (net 6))
 (segment (start 27.604227 -15.2) (end 38.608 -15.2) (width 2) (layer "F.Cu") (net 8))
 (segment (start 12.192 -12.7) (end 25.104227 -12.7) (width 2) (layer "F.Cu") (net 8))
 (segment (start 25.104227 -12.7) (end 27.604227 -15.2) (width 2) (layer "F.Cu") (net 8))
 (segment (start 24.351523 -15.2) (end 27.479523 -18.328) (width 2) (layer "F.Cu") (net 9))
 (segment (start 12.192 -15.2) (end 24.351523 -15.2) (width 2) (layer "F.Cu") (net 9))
 (segment (start 27.479523 -18.328) (end 34.358 -18.328) (width 2) (layer "F.Cu") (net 9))
 (segment (start 34.358 -18.328) (end 38.608 -18.328) (width 2) (layer "F.Cu") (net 9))
 (segment (start 38.608 -12.7) (end 36.346001 -12.7) (width 2) (layer "F.Cu") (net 10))
 (segment (start 15.748 -3.048) (end 15.748 -8.128) (width 1.5) (layer "F.Cu") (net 10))
 (segment (start 20.828 -8.128) (end 20.828 -3.048) (width 1.5) (layer "F.Cu") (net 10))
 (segment (start 15.748 -8.128) (end 20.828 -8.128) (width 1.5) (layer "F.Cu") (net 10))
 (segment (start 19.812 -37.846) (end 19.812 -35.306) (width 2) (layer "F.Cu") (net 10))
 (segment (start 20.828 -3.048) (end 15.748 -3.048) (width 1.5) (layer "F.Cu") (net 10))
 (segment (start 31.496 -9.652) (end 31.496 -12.7) (width 2) (layer "F.Cu") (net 10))
 (via (at 31.496 -12.7) (size 0.8) (drill 0.4) (layers "F.Cu" "B.Cu") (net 10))
 (via (at 36.068 -12.7) (size 0.8) (drill 0.4) (layers "F.Cu" "B.Cu") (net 10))
 (segment (start 20.32 -12.7) (end 19.812 -13.208) (width 2) (layer "B.Cu") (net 10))
 (segment (start 31.496 -12.7) (end 36.068 -12.7) (width 2) (layer "B.Cu") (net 10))
 (segment (start 20.828 -8.128) (end 20.828 -12.192) (width 2) (layer "B.Cu") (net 10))
 (segment (start 19.812 -35.306) (end 19.812 -13.208) (width 2) (layer "B.Cu") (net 10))
 (segment (start 20.828 -12.192) (end 19.812 -13.208) (width 2) (layer "B.Cu") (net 10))
 (segment (start 31.496 -12.7) (end 20.32 -12.7) (width 2) (layer "B.Cu") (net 10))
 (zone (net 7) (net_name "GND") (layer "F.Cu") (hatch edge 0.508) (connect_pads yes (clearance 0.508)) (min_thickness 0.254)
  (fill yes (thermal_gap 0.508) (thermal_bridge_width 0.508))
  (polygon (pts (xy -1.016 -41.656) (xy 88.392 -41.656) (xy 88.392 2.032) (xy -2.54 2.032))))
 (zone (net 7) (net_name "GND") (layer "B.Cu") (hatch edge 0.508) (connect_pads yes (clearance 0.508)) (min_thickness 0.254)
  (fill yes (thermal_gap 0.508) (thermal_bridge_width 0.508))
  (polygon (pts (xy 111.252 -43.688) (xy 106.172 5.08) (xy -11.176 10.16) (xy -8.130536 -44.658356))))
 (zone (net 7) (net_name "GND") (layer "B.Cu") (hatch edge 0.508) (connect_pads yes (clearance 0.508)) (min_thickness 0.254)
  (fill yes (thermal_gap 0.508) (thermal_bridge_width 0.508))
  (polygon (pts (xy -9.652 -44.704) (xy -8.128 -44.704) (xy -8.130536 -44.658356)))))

